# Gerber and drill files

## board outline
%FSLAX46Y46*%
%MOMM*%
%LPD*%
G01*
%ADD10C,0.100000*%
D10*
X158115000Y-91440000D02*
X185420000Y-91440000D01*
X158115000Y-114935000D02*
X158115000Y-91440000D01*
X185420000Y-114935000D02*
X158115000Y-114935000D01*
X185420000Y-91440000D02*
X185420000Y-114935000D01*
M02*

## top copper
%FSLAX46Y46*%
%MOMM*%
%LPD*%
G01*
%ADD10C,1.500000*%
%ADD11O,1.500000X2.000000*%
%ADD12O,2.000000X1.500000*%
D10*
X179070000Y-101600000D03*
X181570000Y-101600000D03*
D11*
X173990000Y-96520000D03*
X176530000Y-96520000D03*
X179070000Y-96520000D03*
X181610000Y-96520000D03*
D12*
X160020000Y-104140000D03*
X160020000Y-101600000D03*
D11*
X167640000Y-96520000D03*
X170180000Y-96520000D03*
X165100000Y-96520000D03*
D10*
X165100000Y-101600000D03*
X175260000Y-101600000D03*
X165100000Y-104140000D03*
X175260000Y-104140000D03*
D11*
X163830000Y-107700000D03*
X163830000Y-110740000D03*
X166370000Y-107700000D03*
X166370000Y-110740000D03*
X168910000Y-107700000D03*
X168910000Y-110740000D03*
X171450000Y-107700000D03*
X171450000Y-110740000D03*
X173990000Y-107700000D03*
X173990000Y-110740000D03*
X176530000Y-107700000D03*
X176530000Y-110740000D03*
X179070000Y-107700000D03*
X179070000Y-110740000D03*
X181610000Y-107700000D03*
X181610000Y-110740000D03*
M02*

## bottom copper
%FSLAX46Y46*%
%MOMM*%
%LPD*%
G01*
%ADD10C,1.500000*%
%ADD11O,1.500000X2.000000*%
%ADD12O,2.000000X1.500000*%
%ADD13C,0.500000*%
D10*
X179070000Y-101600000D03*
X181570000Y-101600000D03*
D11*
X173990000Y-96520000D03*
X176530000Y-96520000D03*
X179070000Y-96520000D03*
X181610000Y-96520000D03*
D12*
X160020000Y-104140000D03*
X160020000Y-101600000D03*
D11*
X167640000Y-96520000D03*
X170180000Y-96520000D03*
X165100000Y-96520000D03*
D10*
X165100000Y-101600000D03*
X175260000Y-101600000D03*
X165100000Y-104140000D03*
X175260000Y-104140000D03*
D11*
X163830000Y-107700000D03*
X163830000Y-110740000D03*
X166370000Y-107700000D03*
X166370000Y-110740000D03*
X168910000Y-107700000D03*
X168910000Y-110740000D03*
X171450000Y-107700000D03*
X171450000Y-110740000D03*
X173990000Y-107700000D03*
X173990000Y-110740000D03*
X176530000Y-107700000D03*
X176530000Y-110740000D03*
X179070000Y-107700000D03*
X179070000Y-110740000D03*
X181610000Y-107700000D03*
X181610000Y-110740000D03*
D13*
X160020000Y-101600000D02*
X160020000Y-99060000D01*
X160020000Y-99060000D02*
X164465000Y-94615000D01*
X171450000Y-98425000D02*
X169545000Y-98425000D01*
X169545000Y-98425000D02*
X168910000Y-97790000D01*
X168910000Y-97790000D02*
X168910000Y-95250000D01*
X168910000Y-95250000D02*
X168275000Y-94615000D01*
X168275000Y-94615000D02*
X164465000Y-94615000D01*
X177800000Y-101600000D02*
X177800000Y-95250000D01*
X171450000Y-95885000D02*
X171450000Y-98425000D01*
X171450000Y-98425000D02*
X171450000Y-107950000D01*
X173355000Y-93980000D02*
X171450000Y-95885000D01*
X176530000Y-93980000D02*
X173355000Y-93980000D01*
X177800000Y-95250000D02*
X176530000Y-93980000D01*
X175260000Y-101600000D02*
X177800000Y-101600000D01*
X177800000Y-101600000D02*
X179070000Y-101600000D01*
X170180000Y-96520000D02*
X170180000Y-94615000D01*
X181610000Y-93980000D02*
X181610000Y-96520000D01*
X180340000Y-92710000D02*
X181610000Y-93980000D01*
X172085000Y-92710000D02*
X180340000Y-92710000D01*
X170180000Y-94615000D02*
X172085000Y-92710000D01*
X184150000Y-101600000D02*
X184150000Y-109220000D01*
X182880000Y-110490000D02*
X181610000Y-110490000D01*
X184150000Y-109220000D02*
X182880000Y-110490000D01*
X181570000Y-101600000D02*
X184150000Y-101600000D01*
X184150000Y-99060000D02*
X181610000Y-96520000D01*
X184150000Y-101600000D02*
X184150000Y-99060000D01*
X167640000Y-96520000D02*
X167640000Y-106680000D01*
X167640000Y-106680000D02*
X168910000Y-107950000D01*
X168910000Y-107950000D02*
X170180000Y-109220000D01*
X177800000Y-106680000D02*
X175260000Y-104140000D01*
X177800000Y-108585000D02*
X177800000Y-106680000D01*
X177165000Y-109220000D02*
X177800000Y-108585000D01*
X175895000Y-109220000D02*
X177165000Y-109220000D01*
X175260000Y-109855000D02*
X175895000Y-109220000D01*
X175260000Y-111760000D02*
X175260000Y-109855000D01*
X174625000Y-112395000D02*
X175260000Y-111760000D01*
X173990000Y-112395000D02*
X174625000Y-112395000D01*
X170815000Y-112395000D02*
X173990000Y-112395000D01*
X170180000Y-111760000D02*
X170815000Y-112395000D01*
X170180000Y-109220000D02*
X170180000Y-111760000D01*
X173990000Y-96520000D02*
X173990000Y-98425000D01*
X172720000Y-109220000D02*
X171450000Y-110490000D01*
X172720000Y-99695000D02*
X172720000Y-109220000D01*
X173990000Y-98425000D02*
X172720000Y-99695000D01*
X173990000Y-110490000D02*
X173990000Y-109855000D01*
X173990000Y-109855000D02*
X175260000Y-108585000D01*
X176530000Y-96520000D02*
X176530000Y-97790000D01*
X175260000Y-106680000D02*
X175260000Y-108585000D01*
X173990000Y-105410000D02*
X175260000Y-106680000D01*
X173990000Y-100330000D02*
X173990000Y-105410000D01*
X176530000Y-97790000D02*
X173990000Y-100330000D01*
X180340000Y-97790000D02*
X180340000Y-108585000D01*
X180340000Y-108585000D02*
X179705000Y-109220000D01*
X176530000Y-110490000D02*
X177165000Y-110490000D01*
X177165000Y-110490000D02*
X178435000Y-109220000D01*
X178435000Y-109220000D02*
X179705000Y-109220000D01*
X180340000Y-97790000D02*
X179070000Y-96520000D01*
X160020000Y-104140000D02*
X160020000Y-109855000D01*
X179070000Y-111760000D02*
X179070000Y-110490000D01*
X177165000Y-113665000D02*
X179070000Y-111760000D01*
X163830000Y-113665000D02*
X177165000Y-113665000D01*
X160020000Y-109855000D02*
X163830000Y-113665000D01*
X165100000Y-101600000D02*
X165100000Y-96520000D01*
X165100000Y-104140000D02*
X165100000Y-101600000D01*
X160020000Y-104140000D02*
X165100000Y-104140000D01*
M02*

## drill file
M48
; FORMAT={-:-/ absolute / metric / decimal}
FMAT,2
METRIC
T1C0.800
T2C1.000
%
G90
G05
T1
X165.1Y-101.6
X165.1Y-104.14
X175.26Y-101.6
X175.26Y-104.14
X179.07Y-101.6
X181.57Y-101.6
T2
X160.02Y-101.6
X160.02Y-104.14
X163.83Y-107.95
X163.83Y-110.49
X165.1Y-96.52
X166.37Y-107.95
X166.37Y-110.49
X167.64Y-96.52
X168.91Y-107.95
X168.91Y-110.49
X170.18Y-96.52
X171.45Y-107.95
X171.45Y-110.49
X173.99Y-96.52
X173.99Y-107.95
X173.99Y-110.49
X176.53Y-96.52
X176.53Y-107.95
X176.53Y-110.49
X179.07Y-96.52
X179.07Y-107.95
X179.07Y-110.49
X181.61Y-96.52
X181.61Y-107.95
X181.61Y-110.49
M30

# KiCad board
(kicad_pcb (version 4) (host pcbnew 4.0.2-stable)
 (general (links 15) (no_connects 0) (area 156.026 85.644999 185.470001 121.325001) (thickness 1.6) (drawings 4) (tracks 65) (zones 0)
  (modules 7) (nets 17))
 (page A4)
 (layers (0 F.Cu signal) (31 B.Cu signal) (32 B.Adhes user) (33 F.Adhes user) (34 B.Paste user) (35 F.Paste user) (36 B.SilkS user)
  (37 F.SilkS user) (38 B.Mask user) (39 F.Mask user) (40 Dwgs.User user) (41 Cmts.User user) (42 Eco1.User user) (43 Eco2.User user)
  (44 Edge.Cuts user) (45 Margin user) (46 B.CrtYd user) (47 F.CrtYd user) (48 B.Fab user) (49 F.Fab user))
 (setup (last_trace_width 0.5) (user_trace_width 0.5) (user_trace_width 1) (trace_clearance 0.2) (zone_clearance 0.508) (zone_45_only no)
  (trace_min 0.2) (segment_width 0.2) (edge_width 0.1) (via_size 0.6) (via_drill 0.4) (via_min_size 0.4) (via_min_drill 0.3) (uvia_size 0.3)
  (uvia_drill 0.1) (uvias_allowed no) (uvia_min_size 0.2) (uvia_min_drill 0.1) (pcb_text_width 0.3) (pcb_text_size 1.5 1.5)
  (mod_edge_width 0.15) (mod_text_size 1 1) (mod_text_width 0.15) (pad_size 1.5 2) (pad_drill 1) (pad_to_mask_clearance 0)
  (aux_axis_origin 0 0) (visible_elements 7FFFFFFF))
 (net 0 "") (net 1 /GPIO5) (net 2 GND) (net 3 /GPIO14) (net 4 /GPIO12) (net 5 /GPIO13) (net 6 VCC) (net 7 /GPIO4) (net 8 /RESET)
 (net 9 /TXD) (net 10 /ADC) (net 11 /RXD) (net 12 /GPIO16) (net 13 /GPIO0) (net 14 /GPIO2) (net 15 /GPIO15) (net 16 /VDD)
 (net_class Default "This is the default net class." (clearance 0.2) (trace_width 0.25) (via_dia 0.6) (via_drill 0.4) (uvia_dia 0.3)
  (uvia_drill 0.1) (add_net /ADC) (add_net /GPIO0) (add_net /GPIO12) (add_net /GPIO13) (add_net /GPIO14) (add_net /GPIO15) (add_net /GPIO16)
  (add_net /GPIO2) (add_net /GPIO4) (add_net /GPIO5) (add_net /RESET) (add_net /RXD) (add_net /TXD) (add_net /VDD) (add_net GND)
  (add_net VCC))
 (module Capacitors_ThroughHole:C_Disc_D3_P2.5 (layer F.Cu) (at 179.07 101.6)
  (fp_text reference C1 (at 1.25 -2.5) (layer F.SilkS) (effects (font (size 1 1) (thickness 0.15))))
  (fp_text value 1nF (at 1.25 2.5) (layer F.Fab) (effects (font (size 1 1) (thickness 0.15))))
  (pad 1 thru_hole circle (at 0 0) (size 1.5 1.5) (drill 0.8) (layers *.Cu *.Mask) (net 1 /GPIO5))
  (pad 2 thru_hole circle (at 2.5 0) (size 1.5 1.5) (drill 0.8) (layers *.Cu *.Mask) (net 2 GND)))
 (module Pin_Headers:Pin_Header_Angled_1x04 (layer F.Cu) (at 173.99 96.52 90)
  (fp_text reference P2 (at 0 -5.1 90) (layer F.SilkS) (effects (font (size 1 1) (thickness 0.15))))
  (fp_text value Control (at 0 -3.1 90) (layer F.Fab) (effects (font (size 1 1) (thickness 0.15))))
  (pad 1 thru_hole oval (at 0 0 90) (size 2 1.5) (drill 1) (layers *.Cu *.Mask) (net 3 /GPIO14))
  (pad 2 thru_hole oval (at 0 2.54 90) (size 2 1.5) (drill 1) (layers *.Cu *.Mask) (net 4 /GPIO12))
  (pad 3 thru_hole oval (at 0 5.08 90) (size 2 1.5) (drill 1) (layers *.Cu *.Mask) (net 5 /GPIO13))
  (pad 4 thru_hole oval (at 0 7.62 90) (size 2 1.5) (drill 1) (layers *.Cu *.Mask) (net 2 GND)))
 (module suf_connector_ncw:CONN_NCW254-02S (layer F.Cu) (at 160.02 102.87 90)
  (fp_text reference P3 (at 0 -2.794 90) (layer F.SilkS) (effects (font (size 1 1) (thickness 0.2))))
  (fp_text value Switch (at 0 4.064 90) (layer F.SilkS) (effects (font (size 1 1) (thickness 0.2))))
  (pad 1 thru_hole oval (at -1.27 0 90) (size 1.5 2) (drill 1) (layers *.Cu *.Mask F.SilkS) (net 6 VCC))
  (pad 2 thru_hole oval (at 1.27 0 90) (size 1.5 2) (drill 1) (layers *.Cu *.Mask F.SilkS) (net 1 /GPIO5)))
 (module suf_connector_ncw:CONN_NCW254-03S (layer F.Cu) (at 167.64 96.52)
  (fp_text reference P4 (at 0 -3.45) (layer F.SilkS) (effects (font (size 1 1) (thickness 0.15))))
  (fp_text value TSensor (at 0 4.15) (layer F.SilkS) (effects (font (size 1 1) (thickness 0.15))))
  (pad 2 thru_hole oval (at 0 0) (size 1.5 2) (drill 1) (layers *.Cu *.Mask) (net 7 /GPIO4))
  (pad 3 thru_hole oval (at 2.54 0) (size 1.5 2) (drill 1) (layers *.Cu *.Mask) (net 2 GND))
  (pad 1 thru_hole oval (at -2.54 0) (size 1.5 2) (drill 1) (layers *.Cu *.Mask) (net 6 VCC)))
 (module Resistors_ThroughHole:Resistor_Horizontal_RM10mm (layer F.Cu) (at 165.1 101.6)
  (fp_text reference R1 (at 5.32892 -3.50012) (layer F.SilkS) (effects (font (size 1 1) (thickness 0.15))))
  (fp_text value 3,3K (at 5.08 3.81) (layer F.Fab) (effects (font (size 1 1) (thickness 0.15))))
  (pad 1 thru_hole circle (at 0 0) (size 1.5 1.5) (drill 0.8) (layers *.Cu *.SilkS *.Mask) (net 6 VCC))
  (pad 2 thru_hole circle (at 10.16 0) (size 1.5 1.5) (drill 0.8) (layers *.Cu *.SilkS *.Mask) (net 1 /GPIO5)))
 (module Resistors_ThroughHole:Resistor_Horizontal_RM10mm (layer F.Cu) (at 165.1 104.14)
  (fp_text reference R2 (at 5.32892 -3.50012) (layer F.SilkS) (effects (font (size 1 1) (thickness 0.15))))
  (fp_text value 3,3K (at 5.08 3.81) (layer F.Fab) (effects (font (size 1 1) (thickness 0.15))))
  (pad 1 thru_hole circle (at 0 0) (size 1.5 1.5) (drill 0.8) (layers *.Cu *.SilkS *.Mask) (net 6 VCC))
  (pad 2 thru_hole circle (at 10.16 0) (size 1.5 1.5) (drill 0.8) (layers *.Cu *.SilkS *.Mask) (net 7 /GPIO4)))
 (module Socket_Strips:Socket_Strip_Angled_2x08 (layer F.Cu) (at 163.83 107.95)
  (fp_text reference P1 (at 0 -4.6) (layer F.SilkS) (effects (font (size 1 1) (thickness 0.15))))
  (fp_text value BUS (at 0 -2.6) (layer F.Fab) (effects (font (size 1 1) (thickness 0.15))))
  (pad 1 thru_hole oval (at 0 0) (size 1.5 2) (drill 1 (offset 0 -0.25)) (layers *.Cu *.Mask) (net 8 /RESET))
  (pad 2 thru_hole oval (at 0 2.54) (size 1.5 2) (drill 1 (offset 0 0.25)) (layers *.Cu *.Mask) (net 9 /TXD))
  (pad 3 thru_hole oval (at 2.54 0) (size 1.5 2) (drill 1 (offset 0 -0.25)) (layers *.Cu *.Mask) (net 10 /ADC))
  (pad 4 thru_hole oval (at 2.54 2.54) (size 1.5 2) (drill 1 (offset 0 0.25)) (layers *.Cu *.Mask) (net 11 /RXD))
  (pad 5 thru_hole oval (at 5.08 0) (size 1.5 2) (drill 1 (offset 0 -0.25)) (layers *.Cu *.Mask) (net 7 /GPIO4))
  (pad 6 thru_hole oval (at 5.08 2.54) (size 1.5 2) (drill 1 (offset 0 0.25)) (layers *.Cu *.Mask) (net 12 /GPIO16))
  (pad 7 thru_hole oval (at 7.62 0) (size 1.5 2) (drill 1 (offset 0 -0.25)) (layers *.Cu *.Mask) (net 1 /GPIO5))
  (pad 8 thru_hole oval (at 7.62 2.54) (size 1.5 2) (drill 1 (offset 0 0.25)) (layers *.Cu *.Mask) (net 3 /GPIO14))
  (pad 9 thru_hole oval (at 10.16 0) (size 1.5 2) (drill 1 (offset 0 -0.25)) (layers *.Cu *.Mask) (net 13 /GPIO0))
  (pad 10 thru_hole oval (at 10.16 2.54) (size 1.5 2) (drill 1 (offset 0 0.25)) (layers *.Cu *.Mask) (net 4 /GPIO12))
  (pad 11 thru_hole oval (at 12.7 0) (size 1.5 2) (drill 1 (offset 0 -0.25)) (layers *.Cu *.Mask) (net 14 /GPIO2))
  (pad 12 thru_hole oval (at 12.7 2.54) (size 1.5 2) (drill 1 (offset 0 0.25)) (layers *.Cu *.Mask) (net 5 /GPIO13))
  (pad 13 thru_hole oval (at 15.24 0) (size 1.5 2) (drill 1 (offset 0 -0.25)) (layers *.Cu *.Mask) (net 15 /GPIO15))
  (pad 14 thru_hole oval (at 15.24 2.54) (size 1.5 2) (drill 1 (offset 0 0.25)) (layers *.Cu *.Mask) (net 6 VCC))
  (pad 15 thru_hole oval (at 17.78 0) (size 1.5 2) (drill 1 (offset 0 -0.25)) (layers *.Cu *.Mask) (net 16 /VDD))
  (pad 16 thru_hole oval (at 17.78 2.54) (size 1.5 2) (drill 1 (offset 0 0.25)) (layers *.Cu *.Mask) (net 2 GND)))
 (gr_line (start 158.115 91.44) (end 185.42 91.44) (angle 90) (layer Edge.Cuts) (width 0.1))
 (gr_line (start 158.115 114.935) (end 158.115 91.44) (angle 90) (layer Edge.Cuts) (width 0.1))
 (gr_line (start 185.42 114.935) (end 158.115 114.935) (angle 90) (layer Edge.Cuts) (width 0.1))
 (gr_line (start 185.42 91.44) (end 185.42 114.935) (angle 90) (layer Edge.Cuts) (width 0.1))
 (segment (start 160.02 101.6) (end 160.02 99.06) (width 0.5) (layer B.Cu) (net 1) (status 400000))
 (segment (start 160.02 99.06) (end 164.465 94.615) (width 0.5) (layer B.Cu) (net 1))
 (segment (start 171.45 98.425) (end 169.545 98.425) (width 0.5) (layer B.Cu) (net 1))
 (segment (start 169.545 98.425) (end 168.91 97.79) (width 0.5) (layer B.Cu) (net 1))
 (segment (start 168.91 97.79) (end 168.91 95.25) (width 0.5) (layer B.Cu) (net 1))
 (segment (start 168.91 95.25) (end 168.275 94.615) (width 0.5) (layer B.Cu) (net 1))
 (segment (start 168.275 94.615) (end 164.465 94.615) (width 0.5) (layer B.Cu) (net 1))
 (segment (start 177.8 101.6) (end 177.8 95.25) (width 0.5) (layer B.Cu) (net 1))
 (segment (start 171.45 95.885) (end 171.45 98.425) (width 0.5) (layer B.Cu) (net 1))
 (segment (start 171.45 98.425) (end 171.45 107.95) (width 0.5) (layer B.Cu) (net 1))
 (segment (start 173.355 93.98) (end 171.45 95.885) (width 0.5) (layer B.Cu) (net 1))
 (segment (start 176.53 93.98) (end 173.355 93.98) (width 0.5) (layer B.Cu) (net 1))
 (segment (start 177.8 95.25) (end 176.53 93.98) (width 0.5) (layer B.Cu) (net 1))
 (segment (start 175.26 101.6) (end 177.8 101.6) (width 0.5) (layer B.Cu) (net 1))
 (segment (start 177.8 101.6) (end 179.07 101.6) (width 0.5) (layer B.Cu) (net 1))
 (segment (start 170.18 96.52) (end 170.18 94.615) (width 0.5) (layer B.Cu) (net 2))
 (segment (start 181.61 93.98) (end 181.61 96.52) (width 0.5) (layer B.Cu) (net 2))
 (segment (start 180.34 92.71) (end 181.61 93.98) (width 0.5) (layer B.Cu) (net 2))
 (segment (start 172.085 92.71) (end 180.34 92.71) (width 0.5) (layer B.Cu) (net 2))
 (segment (start 170.18 94.615) (end 172.085 92.71) (width 0.5) (layer B.Cu) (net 2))
 (segment (start 184.15 101.6) (end 184.15 109.22) (width 0.5) (layer B.Cu) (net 2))
 (segment (start 182.88 110.49) (end 181.61 110.49) (width 0.5) (layer B.Cu) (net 2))
 (segment (start 184.15 109.22) (end 182.88 110.49) (width 0.5) (layer B.Cu) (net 2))
 (segment (start 181.57 101.6) (end 184.15 101.6) (width 0.5) (layer B.Cu) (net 2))
 (segment (start 184.15 99.06) (end 181.61 96.52) (width 0.5) (layer B.Cu) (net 2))
 (segment (start 184.15 101.6) (end 184.15 99.06) (width 0.5) (layer B.Cu) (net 2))
 (segment (start 167.64 96.52) (end 167.64 106.68) (width 0.5) (layer B.Cu) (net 7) (status 400000))
 (segment (start 167.64 106.68) (end 168.91 107.95) (width 0.5) (layer B.Cu) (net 7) (status 800000))
 (segment (start 168.91 107.95) (end 170.18 109.22) (width 0.5) (layer B.Cu) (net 7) (status 400000))
 (segment (start 177.8 106.68) (end 175.26 104.14) (width 0.5) (layer B.Cu) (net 7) (status 800000))
 (segment (start 177.8 108.585) (end 177.8 106.68) (width 0.5) (layer B.Cu) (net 7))
 (segment (start 177.165 109.22) (end 177.8 108.585) (width 0.5) (layer B.Cu) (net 7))
 (segment (start 175.895 109.22) (end 177.165 109.22) (width 0.5) (layer B.Cu) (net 7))
 (segment (start 175.26 109.855) (end 175.895 109.22) (width 0.5) (layer B.Cu) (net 7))
 (segment (start 175.26 111.76) (end 175.26 109.855) (width 0.5) (layer B.Cu) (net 7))
 (segment (start 174.625 112.395) (end 175.26 111.76) (width 0.5) (layer B.Cu) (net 7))
 (segment (start 173.99 112.395) (end 174.625 112.395) (width 0.5) (layer B.Cu) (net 7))
 (segment (start 170.815 112.395) (end 173.99 112.395) (width 0.5) (layer B.Cu) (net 7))
 (segment (start 170.18 111.76) (end 170.815 112.395) (width 0.5) (layer B.Cu) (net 7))
 (segment (start 170.18 109.22) (end 170.18 111.76) (width 0.5) (layer B.Cu) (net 7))
 (segment (start 173.99 96.52) (end 173.99 98.425) (width 0.5) (layer B.Cu) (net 3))
 (segment (start 172.72 109.22) (end 171.45 110.49) (width 0.5) (layer B.Cu) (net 3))
 (segment (start 172.72 99.695) (end 172.72 109.22) (width 0.5) (layer B.Cu) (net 3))
 (segment (start 173.99 98.425) (end 172.72 99.695) (width 0.5) (layer B.Cu) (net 3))
 (segment (start 173.99 110.49) (end 173.99 109.855) (width 0.5) (layer B.Cu) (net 4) (status C00000))
 (segment (start 173.99 109.855) (end 175.26 108.585) (width 0.5) (layer B.Cu) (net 4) (status 400000))
 (segment (start 176.53 96.52) (end 176.53 97.79) (width 0.5) (layer B.Cu) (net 4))
 (segment (start 175.26 106.68) (end 175.26 108.585) (width 0.5) (layer B.Cu) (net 4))
 (segment (start 173.99 105.41) (end 175.26 106.68) (width 0.5) (layer B.Cu) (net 4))
 (segment (start 173.99 100.33) (end 173.99 105.41) (width 0.5) (layer B.Cu) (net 4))
 (segment (start 176.53 97.79) (end 173.99 100.33) (width 0.5) (layer B.Cu) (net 4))
 (segment (start 180.34 97.79) (end 180.34 108.585) (width 0.5) (layer B.Cu) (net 5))
 (segment (start 180.34 108.585) (end 179.705 109.22) (width 0.5) (layer B.Cu) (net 5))
 (segment (start 176.53 110.49) (end 177.165 110.49) (width 0.5) (layer B.Cu) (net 5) (status C00000))
 (segment (start 177.165 110.49) (end 178.435 109.22) (width 0.5) (layer B.Cu) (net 5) (status 400000))
 (segment (start 178.435 109.22) (end 179.705 109.22) (width 0.5) (layer B.Cu) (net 5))
 (segment (start 180.34 97.79) (end 179.07 96.52) (width 0.5) (layer B.Cu) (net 5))
 (segment (start 160.02 104.14) (end 160.02 109.855) (width 0.5) (layer B.Cu) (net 6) (status 400000))
 (segment (start 179.07 111.76) (end 179.07 110.49) (width 0.5) (layer B.Cu) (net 6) (status 800000))
 (segment (start 177.165 113.665) (end 179.07 111.76) (width 0.5) (layer B.Cu) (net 6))
 (segment (start 163.83 113.665) (end 177.165 113.665) (width 0.5) (layer B.Cu) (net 6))
 (segment (start 160.02 109.855) (end 163.83 113.665) (width 0.5) (layer B.Cu) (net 6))
 (segment (start 165.1 101.6) (end 165.1 96.52) (width 0.5) (layer B.Cu) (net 6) (status C00000))
 (segment (start 165.1 104.14) (end 165.1 101.6) (width 0.5) (layer B.Cu) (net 6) (status C00000))
 (segment (start 160.02 104.14) (end 165.1 104.14) (width 0.5) (layer B.Cu) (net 6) (status C00000)))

